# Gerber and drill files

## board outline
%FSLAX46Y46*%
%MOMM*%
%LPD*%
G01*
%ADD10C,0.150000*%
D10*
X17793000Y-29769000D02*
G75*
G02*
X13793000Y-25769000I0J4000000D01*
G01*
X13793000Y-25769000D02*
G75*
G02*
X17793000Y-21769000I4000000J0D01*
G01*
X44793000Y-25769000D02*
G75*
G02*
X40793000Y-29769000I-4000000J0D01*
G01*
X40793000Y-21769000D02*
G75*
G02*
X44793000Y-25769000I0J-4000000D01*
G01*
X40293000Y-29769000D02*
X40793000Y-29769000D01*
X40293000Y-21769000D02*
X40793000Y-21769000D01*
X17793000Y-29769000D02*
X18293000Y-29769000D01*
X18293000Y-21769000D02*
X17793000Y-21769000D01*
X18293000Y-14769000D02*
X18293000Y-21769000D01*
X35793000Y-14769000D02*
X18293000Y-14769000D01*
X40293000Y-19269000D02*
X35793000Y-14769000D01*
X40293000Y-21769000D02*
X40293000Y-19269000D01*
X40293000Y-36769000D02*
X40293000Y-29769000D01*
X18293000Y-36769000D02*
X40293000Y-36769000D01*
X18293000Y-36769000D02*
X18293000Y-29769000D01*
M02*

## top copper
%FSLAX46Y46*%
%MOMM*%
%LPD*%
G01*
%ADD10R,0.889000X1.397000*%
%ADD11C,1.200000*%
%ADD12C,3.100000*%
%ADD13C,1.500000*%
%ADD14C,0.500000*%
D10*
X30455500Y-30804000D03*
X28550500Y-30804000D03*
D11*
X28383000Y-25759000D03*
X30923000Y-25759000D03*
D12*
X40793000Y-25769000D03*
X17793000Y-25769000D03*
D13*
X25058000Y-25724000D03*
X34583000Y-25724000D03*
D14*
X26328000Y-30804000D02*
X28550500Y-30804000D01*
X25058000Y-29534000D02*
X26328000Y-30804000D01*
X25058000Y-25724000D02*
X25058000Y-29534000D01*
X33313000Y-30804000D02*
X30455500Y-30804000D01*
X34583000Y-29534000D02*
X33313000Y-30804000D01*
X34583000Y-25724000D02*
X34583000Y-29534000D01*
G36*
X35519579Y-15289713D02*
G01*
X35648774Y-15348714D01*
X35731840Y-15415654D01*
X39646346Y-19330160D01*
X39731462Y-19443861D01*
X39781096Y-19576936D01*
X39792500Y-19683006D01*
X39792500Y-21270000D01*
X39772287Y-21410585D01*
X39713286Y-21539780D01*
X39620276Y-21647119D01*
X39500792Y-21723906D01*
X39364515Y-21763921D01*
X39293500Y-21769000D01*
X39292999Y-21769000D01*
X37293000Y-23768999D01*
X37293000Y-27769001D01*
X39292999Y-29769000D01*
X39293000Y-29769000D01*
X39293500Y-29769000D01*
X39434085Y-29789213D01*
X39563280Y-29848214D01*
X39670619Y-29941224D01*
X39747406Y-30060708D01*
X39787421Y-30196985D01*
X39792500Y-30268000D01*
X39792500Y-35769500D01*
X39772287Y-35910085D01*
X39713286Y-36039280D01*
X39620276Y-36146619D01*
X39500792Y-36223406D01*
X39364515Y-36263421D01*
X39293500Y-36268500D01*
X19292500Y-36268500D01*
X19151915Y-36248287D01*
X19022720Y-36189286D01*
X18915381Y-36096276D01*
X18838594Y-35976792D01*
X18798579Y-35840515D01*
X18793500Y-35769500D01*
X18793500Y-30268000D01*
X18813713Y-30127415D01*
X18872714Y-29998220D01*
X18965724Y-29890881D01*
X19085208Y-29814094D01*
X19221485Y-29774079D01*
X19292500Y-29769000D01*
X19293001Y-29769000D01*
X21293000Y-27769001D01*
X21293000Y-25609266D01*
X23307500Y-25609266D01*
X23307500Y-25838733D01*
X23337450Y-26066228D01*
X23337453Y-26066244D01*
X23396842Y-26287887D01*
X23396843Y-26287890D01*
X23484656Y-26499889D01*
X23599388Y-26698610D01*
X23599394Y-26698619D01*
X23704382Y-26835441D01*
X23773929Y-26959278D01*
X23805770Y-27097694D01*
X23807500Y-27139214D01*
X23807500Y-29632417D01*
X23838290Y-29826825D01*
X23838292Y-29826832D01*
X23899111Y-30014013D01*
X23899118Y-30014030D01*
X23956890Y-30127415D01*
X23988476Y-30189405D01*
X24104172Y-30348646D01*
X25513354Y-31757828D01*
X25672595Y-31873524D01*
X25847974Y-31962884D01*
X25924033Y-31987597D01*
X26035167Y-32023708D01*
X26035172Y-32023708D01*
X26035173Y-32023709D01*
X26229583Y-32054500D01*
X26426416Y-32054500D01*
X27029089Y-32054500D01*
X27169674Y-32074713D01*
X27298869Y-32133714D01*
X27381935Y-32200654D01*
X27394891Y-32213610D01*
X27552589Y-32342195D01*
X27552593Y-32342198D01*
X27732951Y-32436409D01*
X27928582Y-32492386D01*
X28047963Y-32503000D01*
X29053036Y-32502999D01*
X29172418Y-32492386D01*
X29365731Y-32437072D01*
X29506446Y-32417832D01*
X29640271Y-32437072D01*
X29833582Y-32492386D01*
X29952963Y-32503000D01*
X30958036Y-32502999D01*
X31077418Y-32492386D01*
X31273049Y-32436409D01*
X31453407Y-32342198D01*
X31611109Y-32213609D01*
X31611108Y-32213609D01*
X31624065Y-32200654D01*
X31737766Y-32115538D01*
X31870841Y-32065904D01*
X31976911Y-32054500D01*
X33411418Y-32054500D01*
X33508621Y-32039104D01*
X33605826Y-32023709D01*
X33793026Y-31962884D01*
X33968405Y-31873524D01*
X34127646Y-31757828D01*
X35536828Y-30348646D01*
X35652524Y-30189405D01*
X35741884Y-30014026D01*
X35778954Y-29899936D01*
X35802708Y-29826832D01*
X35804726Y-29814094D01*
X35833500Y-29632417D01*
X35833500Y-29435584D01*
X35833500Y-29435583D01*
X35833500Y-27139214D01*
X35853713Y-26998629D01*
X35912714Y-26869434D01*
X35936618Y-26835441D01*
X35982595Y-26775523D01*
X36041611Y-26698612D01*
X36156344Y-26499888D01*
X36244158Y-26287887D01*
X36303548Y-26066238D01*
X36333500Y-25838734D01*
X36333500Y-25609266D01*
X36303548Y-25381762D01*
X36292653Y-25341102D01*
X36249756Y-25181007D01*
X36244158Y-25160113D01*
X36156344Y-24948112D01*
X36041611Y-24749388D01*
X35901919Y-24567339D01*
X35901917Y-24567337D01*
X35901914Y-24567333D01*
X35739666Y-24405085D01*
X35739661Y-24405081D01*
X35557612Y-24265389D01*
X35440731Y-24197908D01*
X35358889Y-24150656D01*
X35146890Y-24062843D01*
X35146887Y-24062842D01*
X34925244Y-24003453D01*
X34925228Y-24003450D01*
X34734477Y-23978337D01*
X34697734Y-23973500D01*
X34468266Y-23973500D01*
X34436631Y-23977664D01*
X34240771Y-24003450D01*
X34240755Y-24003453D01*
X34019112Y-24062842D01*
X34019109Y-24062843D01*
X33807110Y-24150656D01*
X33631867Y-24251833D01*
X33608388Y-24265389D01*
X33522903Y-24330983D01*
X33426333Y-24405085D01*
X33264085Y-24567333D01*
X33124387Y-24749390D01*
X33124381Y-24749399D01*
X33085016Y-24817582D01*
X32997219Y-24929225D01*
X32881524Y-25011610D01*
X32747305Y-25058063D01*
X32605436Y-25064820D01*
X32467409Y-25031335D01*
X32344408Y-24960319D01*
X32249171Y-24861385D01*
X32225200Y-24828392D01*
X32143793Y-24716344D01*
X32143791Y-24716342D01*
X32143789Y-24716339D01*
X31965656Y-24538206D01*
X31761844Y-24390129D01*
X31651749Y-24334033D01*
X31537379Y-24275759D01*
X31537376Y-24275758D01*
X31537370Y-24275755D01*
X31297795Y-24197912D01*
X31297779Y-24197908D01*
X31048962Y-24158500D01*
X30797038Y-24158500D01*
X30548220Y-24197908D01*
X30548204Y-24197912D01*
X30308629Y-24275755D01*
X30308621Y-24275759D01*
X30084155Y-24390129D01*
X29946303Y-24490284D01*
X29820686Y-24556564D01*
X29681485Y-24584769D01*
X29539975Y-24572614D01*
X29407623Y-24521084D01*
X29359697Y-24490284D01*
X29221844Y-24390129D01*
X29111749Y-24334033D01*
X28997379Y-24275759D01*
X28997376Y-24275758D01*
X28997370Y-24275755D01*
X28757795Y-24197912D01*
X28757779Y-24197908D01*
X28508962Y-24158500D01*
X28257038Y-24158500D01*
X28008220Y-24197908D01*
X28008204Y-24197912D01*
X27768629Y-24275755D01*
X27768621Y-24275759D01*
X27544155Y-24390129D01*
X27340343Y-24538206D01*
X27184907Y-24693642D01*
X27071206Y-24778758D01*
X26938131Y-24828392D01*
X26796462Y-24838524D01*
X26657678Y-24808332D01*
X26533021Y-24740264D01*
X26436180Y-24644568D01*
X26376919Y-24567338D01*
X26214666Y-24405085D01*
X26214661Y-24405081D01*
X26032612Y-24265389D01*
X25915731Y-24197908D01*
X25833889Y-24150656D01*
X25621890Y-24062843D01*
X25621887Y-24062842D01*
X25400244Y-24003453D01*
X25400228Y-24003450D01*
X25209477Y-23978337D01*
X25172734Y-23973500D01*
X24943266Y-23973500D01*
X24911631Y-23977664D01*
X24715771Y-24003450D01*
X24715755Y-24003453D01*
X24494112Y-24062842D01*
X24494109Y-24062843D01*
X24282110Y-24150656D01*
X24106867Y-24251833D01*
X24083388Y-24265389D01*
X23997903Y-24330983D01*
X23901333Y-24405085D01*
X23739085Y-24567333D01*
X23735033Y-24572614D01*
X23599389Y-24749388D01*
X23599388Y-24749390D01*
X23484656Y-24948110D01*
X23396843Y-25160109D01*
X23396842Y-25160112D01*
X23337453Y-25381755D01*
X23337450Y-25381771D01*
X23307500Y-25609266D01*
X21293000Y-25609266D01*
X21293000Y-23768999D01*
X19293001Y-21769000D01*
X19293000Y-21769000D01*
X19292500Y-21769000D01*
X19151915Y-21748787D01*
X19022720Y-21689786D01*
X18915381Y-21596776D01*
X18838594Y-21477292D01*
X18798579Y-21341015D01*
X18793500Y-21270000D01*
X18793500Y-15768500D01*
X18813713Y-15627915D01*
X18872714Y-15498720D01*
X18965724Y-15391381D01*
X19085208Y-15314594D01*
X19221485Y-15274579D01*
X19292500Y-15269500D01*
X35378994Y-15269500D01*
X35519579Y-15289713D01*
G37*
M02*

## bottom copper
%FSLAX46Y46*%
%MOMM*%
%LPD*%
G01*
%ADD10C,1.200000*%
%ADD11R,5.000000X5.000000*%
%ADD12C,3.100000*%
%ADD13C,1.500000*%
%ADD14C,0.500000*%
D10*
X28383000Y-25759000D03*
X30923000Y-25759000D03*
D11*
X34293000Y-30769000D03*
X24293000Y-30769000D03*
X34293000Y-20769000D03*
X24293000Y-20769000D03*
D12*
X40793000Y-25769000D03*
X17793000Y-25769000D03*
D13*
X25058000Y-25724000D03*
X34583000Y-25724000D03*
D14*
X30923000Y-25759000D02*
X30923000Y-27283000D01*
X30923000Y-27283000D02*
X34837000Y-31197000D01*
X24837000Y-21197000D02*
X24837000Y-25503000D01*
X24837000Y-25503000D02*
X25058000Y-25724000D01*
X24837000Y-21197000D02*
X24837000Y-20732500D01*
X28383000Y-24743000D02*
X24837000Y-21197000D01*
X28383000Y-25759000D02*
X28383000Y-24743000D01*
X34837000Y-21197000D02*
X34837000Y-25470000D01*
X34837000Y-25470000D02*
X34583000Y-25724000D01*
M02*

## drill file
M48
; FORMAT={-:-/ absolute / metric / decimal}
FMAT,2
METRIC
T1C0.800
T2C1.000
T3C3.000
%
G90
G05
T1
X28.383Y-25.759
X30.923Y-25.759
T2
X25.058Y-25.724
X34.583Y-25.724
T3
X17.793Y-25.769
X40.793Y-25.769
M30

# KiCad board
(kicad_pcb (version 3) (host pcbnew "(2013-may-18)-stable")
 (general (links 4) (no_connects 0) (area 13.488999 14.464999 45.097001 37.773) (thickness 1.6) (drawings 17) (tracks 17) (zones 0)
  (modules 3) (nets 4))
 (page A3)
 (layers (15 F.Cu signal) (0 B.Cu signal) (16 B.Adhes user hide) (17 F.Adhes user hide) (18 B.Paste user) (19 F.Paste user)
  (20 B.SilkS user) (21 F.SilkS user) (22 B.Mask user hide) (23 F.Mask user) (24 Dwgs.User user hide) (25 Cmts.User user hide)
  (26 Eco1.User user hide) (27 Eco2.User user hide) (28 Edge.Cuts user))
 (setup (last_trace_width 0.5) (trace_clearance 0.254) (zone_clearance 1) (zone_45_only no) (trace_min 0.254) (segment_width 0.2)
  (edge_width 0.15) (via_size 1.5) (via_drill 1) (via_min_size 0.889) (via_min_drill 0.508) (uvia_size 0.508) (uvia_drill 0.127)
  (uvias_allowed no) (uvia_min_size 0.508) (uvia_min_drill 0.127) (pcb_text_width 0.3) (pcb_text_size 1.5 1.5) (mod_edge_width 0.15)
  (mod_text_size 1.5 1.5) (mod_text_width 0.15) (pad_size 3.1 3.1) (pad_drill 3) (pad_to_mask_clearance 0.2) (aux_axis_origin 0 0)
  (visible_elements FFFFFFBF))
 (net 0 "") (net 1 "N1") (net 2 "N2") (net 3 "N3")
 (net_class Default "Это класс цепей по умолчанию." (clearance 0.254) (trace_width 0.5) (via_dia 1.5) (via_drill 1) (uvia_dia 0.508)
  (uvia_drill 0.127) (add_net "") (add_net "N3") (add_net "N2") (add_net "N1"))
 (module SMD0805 (layer F.Cu) (at 29.503 30.804 180)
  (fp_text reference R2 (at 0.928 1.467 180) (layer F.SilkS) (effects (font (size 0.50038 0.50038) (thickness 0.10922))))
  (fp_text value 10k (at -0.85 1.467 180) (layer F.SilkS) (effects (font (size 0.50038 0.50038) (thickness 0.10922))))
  (pad 1 smd rect (at -0.9525 0 180) (size 0.889 1.397) (layers F.Cu F.Paste F.Mask) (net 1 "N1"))
  (pad 2 smd rect (at 0.9525 0 180) (size 0.889 1.397) (layers F.Cu F.Paste F.Mask) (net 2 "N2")))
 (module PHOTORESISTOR (layer F.Cu) (at 28.383 25.759)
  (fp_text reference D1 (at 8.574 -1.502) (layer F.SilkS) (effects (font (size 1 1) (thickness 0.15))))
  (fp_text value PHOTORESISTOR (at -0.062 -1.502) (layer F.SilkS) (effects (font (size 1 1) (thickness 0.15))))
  (pad 2 thru_hole circle (at 0 0) (size 1.2 1.2) (drill 0.8) (layers *.Cu *.Mask F.SilkS) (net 2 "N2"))
  (pad 1 thru_hole circle (at 2.54 0) (size 1.2 1.2) (drill 0.8) (layers *.Cu *.Mask F.SilkS) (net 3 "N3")))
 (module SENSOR (layer B.Cu) (at 40.793 37.269 180)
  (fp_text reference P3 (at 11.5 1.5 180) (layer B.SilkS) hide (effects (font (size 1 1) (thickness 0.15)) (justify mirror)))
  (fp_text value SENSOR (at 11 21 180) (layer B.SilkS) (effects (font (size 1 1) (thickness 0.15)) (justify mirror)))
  (pad 2 smd rect (at 6.5 6.5 180) (size 5 5) (layers B.Cu B.Mask) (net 3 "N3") (solder_mask_margin 0.1))
  (pad 3 smd rect (at 16.5 6.5 180) (size 5 5) (layers B.Cu B.Mask))
  (pad 1 smd rect (at 6.5 16.5 180) (size 5 5) (layers B.Cu B.Mask) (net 1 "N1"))
  (pad 4 smd rect (at 16.5 16.5 180) (size 5 5) (layers B.Cu B.Mask) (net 2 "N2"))
  (pad "" np_thru_hole circle (at 0 11.5 180) (size 3.1 3.1) (drill 3) (layers *.Cu *.Mask B.SilkS))
  (pad "" np_thru_hole circle (at 23 11.5 180) (size 3.1 3.1) (drill 3) (layers *.Cu *.Mask B.SilkS)))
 (gr_arc (start 17.793 25.769) (end 17.793 29.769) (angle 90) (layer Edge.Cuts) (width 0.15))
 (gr_arc (start 17.793 25.769) (end 13.793 25.769) (angle 90) (layer Edge.Cuts) (width 0.15))
 (gr_arc (start 40.793 25.769) (end 44.793 25.769) (angle 90) (layer Edge.Cuts) (width 0.15))
 (gr_arc (start 40.793 25.769) (end 40.793 21.769) (angle 90) (layer Edge.Cuts) (width 0.15))
 (gr_line (start 40.293 29.769) (end 40.793 29.769) (angle 90) (layer Edge.Cuts) (width 0.15))
 (gr_line (start 40.293 21.769) (end 40.793 21.769) (angle 90) (layer Edge.Cuts) (width 0.15))
 (gr_line (start 17.793 29.769) (end 18.293 29.769) (angle 90) (layer Edge.Cuts) (width 0.15))
 (gr_line (start 18.293 21.769) (end 17.793 21.769) (angle 90) (layer Edge.Cuts) (width 0.15))
 (gr_line (start 18.293 14.769) (end 18.293 21.769) (angle 90) (layer Edge.Cuts) (width 0.15))
 (gr_line (start 35.793 14.769) (end 18.293 14.769) (angle 90) (layer Edge.Cuts) (width 0.15))
 (gr_line (start 40.293 19.269) (end 35.793 14.769) (angle 90) (layer Edge.Cuts) (width 0.15))
 (gr_line (start 40.293 21.769) (end 40.293 19.269) (angle 90) (layer Edge.Cuts) (width 0.15))
 (gr_line (start 40.293 36.769) (end 40.293 29.769) (angle 90) (layer Edge.Cuts) (width 0.15))
 (gr_line (start 18.293 36.769) (end 40.293 36.769) (angle 90) (layer Edge.Cuts) (width 0.15))
 (gr_line (start 18.293 36.769) (end 18.293 29.769) (angle 90) (layer Edge.Cuts) (width 0.15))
 (segment (start 30.923 25.759) (end 30.923 27.283) (width 0.5) (layer B.Cu) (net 3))
 (segment (start 30.923 27.283) (end 34.837 31.197) (width 0.5) (layer B.Cu) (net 3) (status 20))
 (segment (start 24.837 21.197) (end 24.837 25.503) (width 0.5) (layer B.Cu) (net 2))
 (segment (start 26.328 30.804) (end 28.5505 30.804) (width 0.5) (layer F.Cu) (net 2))
 (segment (start 25.058 29.534) (end 26.328 30.804) (width 0.5) (layer F.Cu) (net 2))
 (segment (start 25.058 25.724) (end 25.058 29.534) (width 0.5) (layer F.Cu) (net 2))
 (via (at 25.058 25.724) (size 1.5) (layers F.Cu B.Cu) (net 2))
 (segment (start 24.837 25.503) (end 25.058 25.724) (width 0.5) (layer B.Cu) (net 2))
 (segment (start 24.837 21.197) (end 24.837 20.7325) (width 0.5) (layer B.Cu) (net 2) (status 30))
 (segment (start 28.383 24.743) (end 24.837 21.197) (width 0.5) (layer B.Cu) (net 2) (status 20))
 (segment (start 28.383 25.759) (end 28.383 24.743) (width 0.5) (layer B.Cu) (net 2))
 (segment (start 34.837 21.197) (end 34.837 25.47) (width 0.5) (layer B.Cu) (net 1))
 (segment (start 33.313 30.804) (end 30.4555 30.804) (width 0.5) (layer F.Cu) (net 1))
 (segment (start 34.583 29.534) (end 33.313 30.804) (width 0.5) (layer F.Cu) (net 1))
 (segment (start 34.583 25.724) (end 34.583 29.534) (width 0.5) (layer F.Cu) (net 1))
 (via (at 34.583 25.724) (size 1.5) (layers F.Cu B.Cu) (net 1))
 (segment (start 34.837 25.47) (end 34.583 25.724) (width 0.5) (layer B.Cu) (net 1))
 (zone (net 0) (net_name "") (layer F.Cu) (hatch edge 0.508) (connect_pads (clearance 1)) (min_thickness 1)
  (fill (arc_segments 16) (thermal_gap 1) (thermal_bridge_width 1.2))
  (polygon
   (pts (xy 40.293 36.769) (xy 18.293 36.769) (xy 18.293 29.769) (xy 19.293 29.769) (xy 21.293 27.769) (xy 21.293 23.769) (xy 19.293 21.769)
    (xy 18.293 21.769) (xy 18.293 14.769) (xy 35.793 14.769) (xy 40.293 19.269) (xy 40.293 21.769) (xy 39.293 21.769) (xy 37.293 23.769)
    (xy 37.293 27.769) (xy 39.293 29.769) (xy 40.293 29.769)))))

